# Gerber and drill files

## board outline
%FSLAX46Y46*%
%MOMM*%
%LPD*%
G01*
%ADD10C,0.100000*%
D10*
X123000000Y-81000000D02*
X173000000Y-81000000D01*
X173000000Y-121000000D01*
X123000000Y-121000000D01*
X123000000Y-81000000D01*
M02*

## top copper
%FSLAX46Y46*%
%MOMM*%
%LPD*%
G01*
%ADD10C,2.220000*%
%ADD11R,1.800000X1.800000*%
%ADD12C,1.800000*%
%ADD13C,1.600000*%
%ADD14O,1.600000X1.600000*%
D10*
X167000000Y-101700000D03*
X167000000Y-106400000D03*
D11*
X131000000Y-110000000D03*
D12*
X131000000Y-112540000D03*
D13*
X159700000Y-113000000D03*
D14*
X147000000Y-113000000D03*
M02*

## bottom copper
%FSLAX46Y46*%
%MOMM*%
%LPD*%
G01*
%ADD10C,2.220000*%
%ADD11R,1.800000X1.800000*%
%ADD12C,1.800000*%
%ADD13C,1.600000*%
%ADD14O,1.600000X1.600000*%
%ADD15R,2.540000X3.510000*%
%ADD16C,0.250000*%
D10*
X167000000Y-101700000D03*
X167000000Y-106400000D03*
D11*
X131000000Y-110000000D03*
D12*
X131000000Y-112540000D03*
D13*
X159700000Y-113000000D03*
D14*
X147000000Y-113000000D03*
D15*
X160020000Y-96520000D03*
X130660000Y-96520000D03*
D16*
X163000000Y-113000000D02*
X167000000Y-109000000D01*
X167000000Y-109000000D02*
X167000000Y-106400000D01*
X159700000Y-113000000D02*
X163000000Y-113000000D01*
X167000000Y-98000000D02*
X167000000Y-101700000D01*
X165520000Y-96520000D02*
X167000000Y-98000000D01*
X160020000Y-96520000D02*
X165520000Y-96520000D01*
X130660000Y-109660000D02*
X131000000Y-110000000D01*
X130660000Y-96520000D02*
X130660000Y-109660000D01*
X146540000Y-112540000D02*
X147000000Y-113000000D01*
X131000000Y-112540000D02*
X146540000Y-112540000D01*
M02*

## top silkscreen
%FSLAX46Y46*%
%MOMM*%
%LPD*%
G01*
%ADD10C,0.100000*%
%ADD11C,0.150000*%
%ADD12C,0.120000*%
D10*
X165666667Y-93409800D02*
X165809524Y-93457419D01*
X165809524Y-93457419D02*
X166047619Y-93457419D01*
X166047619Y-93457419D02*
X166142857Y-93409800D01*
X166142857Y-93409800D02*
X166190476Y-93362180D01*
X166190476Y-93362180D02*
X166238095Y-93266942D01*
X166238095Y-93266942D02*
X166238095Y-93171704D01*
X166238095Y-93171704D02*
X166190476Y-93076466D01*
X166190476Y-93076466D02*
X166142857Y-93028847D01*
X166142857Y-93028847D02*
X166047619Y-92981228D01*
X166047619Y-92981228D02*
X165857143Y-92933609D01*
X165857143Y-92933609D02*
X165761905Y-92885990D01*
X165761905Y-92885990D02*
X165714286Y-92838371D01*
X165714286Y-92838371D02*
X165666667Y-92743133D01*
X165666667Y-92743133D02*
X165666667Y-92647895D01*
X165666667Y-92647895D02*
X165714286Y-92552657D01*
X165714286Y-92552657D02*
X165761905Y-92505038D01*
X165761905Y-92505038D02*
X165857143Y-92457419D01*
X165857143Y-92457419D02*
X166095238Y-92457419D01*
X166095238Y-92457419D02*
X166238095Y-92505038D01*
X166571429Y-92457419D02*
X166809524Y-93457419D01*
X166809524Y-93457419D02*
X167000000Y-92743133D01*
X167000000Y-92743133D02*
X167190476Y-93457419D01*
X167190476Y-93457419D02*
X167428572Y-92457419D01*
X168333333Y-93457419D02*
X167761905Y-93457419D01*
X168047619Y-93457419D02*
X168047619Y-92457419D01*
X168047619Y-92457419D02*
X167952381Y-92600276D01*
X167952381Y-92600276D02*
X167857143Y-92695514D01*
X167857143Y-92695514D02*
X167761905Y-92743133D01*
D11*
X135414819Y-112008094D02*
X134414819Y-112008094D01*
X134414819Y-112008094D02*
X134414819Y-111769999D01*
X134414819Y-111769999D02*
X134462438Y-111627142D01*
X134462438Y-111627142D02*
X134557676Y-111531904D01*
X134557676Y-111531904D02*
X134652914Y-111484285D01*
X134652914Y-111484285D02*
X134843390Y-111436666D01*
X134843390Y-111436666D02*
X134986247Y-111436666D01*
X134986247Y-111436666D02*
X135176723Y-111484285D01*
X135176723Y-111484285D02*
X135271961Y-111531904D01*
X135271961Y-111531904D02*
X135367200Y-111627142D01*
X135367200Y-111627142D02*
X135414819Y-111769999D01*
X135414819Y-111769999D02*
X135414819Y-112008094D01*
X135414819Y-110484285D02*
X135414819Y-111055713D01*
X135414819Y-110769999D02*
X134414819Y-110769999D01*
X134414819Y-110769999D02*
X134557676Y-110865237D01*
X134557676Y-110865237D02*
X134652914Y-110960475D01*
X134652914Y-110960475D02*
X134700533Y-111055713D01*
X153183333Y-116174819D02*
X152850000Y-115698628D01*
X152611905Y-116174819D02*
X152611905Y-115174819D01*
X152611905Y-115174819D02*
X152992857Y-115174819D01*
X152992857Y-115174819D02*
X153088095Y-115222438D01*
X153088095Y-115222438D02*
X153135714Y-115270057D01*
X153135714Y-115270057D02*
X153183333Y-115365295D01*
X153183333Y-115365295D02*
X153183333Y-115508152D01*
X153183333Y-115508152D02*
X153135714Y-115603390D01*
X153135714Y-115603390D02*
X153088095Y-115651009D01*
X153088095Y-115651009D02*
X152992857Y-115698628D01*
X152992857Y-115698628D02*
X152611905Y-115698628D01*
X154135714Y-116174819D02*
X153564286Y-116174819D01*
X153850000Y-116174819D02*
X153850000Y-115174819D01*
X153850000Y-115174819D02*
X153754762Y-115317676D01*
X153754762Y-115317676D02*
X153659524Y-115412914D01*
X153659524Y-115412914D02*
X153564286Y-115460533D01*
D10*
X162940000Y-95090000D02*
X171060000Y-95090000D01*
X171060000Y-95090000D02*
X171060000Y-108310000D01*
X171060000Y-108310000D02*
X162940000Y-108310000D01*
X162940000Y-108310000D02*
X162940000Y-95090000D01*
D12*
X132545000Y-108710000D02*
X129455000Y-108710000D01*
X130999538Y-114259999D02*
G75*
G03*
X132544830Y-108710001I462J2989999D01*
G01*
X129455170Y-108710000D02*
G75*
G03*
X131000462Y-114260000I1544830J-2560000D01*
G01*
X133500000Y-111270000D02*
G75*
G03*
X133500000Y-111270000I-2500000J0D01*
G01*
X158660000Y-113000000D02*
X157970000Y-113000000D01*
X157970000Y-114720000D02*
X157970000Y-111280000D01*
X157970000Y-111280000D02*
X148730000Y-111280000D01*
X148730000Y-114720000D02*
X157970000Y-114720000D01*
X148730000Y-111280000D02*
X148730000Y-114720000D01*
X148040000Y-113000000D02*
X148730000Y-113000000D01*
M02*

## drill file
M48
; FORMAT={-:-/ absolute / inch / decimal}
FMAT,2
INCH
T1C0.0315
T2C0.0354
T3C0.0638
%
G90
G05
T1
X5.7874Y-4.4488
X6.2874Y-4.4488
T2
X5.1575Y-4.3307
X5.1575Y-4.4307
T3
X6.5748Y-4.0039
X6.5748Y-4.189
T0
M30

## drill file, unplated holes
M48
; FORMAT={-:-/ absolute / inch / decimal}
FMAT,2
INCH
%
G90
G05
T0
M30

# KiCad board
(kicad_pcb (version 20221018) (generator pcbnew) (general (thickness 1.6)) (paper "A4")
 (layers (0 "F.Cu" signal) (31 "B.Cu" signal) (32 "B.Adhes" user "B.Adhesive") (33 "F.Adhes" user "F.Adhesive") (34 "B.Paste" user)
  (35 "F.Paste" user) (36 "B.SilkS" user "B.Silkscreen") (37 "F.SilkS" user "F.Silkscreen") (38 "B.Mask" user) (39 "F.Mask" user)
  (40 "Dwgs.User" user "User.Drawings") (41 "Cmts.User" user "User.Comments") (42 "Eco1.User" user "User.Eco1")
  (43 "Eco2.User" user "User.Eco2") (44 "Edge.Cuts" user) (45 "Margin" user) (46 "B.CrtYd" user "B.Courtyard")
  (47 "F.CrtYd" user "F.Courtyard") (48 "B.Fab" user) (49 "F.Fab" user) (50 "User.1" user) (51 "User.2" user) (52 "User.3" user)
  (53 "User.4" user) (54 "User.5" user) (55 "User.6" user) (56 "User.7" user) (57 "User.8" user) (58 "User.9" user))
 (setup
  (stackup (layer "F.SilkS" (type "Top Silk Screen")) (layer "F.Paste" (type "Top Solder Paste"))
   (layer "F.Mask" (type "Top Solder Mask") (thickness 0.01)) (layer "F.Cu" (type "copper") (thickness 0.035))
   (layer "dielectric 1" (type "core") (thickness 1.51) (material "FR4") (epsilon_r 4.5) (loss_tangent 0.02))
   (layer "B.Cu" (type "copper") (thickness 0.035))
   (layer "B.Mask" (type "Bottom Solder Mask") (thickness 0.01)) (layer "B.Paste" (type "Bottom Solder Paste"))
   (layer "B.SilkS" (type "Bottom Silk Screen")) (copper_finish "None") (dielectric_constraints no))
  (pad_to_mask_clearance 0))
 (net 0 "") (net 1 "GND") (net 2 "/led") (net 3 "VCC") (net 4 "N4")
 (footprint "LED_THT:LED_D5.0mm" (layer "F.Cu") (at 131 110 -90)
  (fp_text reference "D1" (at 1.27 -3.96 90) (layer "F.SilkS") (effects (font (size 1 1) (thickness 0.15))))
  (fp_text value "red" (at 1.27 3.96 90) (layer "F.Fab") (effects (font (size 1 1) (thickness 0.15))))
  (fp_line (start -1.29 -1.545) (end -1.29 1.545) (stroke (width 0.12) (type solid)) (layer "F.SilkS"))
  (fp_arc (start -1.29 -1.54483) (mid 2.072002 -2.880433) (end 4.26 0.000462) (stroke (width 0.12) (type solid)) (layer "F.SilkS"))
  (fp_arc (start 4.26 -0.000462) (mid 2.072002 2.880433) (end -1.29 1.54483) (stroke (width 0.12) (type solid)) (layer "F.SilkS"))
  (fp_circle (center 1.27 0) (end 3.77 0) (stroke (width 0.12) (type solid)) (fill none) (layer "F.SilkS"))
  (pad "1" thru_hole rect (at 0 0 270) (size 1.8 1.8) (drill 0.9) (layers "*.Cu" "*.Mask") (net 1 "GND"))
  (pad "2" thru_hole circle (at 2.54 0 270) (size 1.8 1.8) (drill 0.9) (layers "*.Cu" "*.Mask") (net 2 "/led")))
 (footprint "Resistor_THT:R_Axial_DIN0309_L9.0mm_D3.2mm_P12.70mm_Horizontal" (layer "F.Cu") (at 159.7 113 180)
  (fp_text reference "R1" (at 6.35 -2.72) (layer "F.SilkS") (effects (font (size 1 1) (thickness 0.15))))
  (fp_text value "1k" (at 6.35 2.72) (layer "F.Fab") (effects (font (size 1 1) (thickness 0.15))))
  (fp_line (start 1.04 0) (end 1.73 0) (stroke (width 0.12) (type solid)) (layer "F.SilkS"))
  (fp_line (start 1.73 -1.72) (end 1.73 1.72) (stroke (width 0.12) (type solid)) (layer "F.SilkS"))
  (fp_line (start 1.73 1.72) (end 10.97 1.72) (stroke (width 0.12) (type solid)) (layer "F.SilkS"))
  (fp_line (start 10.97 -1.72) (end 1.73 -1.72) (stroke (width 0.12) (type solid)) (layer "F.SilkS"))
  (fp_line (start 10.97 1.72) (end 10.97 -1.72) (stroke (width 0.12) (type solid)) (layer "F.SilkS"))
  (fp_line (start 11.66 0) (end 10.97 0) (stroke (width 0.12) (type solid)) (layer "F.SilkS"))
  (pad "1" thru_hole circle (at 0 0 180) (size 1.6 1.6) (drill 0.8) (layers "*.Cu" "*.Mask") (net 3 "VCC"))
  (pad "2" thru_hole oval (at 12.7 0 180) (size 1.6 1.6) (drill 0.8) (layers "*.Cu" "*.Mask") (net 2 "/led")))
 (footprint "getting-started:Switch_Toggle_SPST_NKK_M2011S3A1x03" (layer "F.Cu") (at 167 97)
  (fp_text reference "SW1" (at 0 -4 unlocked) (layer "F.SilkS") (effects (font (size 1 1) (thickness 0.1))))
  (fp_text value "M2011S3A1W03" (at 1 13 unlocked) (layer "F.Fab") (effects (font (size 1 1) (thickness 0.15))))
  (fp_rect (start -4.06 -1.91) (end 4.06 11.31) (stroke (width 0.1) (type default)) (fill none) (layer "F.SilkS"))
  (pad "2" thru_hole circle (at 0 4.7) (size 2.22 2.22) (drill 1.62) (layers "*.Cu" "*.Mask") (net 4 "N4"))
  (pad "3" thru_hole circle (at 0 9.4) (size 2.22 2.22) (drill 1.62) (layers "*.Cu" "*.Mask") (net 3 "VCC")))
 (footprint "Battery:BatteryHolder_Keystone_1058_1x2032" (layer "B.Cu") (at 145.34 96.52 180)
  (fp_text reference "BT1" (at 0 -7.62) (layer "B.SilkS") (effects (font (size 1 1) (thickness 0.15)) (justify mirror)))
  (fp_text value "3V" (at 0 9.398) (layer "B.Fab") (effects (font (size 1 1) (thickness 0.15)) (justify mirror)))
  (pad "1" smd rect (at -14.68 0 180) (size 2.54 3.51) (layers "B.Cu" "B.Paste" "B.Mask") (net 4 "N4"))
  (pad "2" smd rect (at 14.68 0 180) (size 2.54 3.51) (layers "B.Cu" "B.Paste" "B.Mask") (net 1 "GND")))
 (gr_rect (start 123 81) (end 173 121) (stroke (width 0.1) (type default)) (fill none) (layer "Edge.Cuts"))
 (segment (start 163 113) (end 167 109) (width 0.25) (layer "B.Cu") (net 3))
 (segment (start 167 109) (end 167 106.4) (width 0.25) (layer "B.Cu") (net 3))
 (segment (start 159.7 113) (end 163 113) (width 0.25) (layer "B.Cu") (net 3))
 (segment (start 130.66 109.66) (end 131 110) (width 0.25) (layer "B.Cu") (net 1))
 (segment (start 130.66 96.52) (end 130.66 109.66) (width 0.25) (layer "B.Cu") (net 1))
 (segment (start 146.54 112.54) (end 147 113) (width 0.25) (layer "B.Cu") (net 2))
 (segment (start 131 112.54) (end 146.54 112.54) (width 0.25) (layer "B.Cu") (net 2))
 (segment (start 165.52 96.52) (end 167 98) (width 0.25) (layer "B.Cu") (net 4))
 (segment (start 160.02 96.52) (end 165.52 96.52) (width 0.25) (layer "B.Cu") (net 4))
 (segment (start 167 98) (end 167 101.7) (width 0.25) (layer "B.Cu") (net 4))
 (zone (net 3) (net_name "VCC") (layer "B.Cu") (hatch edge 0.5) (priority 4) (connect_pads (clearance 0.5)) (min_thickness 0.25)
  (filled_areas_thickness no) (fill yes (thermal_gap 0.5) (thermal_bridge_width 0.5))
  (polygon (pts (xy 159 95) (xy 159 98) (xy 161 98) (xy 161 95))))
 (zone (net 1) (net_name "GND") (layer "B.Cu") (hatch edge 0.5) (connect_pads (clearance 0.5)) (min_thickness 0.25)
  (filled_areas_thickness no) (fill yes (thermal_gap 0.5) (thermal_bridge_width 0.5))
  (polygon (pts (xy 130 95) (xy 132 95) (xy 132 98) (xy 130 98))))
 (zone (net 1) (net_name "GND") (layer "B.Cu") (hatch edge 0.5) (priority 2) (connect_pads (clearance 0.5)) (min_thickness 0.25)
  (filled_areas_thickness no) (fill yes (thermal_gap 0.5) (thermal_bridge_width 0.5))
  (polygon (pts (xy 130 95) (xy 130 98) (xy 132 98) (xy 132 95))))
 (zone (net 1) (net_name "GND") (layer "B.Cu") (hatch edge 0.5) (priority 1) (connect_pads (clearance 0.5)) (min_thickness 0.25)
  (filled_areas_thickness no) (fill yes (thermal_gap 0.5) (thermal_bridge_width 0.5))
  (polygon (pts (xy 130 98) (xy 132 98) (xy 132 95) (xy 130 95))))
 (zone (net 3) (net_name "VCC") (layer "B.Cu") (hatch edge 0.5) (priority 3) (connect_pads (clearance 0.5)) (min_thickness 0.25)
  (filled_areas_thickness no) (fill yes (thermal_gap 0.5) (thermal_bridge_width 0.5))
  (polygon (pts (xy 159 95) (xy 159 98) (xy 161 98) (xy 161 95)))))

